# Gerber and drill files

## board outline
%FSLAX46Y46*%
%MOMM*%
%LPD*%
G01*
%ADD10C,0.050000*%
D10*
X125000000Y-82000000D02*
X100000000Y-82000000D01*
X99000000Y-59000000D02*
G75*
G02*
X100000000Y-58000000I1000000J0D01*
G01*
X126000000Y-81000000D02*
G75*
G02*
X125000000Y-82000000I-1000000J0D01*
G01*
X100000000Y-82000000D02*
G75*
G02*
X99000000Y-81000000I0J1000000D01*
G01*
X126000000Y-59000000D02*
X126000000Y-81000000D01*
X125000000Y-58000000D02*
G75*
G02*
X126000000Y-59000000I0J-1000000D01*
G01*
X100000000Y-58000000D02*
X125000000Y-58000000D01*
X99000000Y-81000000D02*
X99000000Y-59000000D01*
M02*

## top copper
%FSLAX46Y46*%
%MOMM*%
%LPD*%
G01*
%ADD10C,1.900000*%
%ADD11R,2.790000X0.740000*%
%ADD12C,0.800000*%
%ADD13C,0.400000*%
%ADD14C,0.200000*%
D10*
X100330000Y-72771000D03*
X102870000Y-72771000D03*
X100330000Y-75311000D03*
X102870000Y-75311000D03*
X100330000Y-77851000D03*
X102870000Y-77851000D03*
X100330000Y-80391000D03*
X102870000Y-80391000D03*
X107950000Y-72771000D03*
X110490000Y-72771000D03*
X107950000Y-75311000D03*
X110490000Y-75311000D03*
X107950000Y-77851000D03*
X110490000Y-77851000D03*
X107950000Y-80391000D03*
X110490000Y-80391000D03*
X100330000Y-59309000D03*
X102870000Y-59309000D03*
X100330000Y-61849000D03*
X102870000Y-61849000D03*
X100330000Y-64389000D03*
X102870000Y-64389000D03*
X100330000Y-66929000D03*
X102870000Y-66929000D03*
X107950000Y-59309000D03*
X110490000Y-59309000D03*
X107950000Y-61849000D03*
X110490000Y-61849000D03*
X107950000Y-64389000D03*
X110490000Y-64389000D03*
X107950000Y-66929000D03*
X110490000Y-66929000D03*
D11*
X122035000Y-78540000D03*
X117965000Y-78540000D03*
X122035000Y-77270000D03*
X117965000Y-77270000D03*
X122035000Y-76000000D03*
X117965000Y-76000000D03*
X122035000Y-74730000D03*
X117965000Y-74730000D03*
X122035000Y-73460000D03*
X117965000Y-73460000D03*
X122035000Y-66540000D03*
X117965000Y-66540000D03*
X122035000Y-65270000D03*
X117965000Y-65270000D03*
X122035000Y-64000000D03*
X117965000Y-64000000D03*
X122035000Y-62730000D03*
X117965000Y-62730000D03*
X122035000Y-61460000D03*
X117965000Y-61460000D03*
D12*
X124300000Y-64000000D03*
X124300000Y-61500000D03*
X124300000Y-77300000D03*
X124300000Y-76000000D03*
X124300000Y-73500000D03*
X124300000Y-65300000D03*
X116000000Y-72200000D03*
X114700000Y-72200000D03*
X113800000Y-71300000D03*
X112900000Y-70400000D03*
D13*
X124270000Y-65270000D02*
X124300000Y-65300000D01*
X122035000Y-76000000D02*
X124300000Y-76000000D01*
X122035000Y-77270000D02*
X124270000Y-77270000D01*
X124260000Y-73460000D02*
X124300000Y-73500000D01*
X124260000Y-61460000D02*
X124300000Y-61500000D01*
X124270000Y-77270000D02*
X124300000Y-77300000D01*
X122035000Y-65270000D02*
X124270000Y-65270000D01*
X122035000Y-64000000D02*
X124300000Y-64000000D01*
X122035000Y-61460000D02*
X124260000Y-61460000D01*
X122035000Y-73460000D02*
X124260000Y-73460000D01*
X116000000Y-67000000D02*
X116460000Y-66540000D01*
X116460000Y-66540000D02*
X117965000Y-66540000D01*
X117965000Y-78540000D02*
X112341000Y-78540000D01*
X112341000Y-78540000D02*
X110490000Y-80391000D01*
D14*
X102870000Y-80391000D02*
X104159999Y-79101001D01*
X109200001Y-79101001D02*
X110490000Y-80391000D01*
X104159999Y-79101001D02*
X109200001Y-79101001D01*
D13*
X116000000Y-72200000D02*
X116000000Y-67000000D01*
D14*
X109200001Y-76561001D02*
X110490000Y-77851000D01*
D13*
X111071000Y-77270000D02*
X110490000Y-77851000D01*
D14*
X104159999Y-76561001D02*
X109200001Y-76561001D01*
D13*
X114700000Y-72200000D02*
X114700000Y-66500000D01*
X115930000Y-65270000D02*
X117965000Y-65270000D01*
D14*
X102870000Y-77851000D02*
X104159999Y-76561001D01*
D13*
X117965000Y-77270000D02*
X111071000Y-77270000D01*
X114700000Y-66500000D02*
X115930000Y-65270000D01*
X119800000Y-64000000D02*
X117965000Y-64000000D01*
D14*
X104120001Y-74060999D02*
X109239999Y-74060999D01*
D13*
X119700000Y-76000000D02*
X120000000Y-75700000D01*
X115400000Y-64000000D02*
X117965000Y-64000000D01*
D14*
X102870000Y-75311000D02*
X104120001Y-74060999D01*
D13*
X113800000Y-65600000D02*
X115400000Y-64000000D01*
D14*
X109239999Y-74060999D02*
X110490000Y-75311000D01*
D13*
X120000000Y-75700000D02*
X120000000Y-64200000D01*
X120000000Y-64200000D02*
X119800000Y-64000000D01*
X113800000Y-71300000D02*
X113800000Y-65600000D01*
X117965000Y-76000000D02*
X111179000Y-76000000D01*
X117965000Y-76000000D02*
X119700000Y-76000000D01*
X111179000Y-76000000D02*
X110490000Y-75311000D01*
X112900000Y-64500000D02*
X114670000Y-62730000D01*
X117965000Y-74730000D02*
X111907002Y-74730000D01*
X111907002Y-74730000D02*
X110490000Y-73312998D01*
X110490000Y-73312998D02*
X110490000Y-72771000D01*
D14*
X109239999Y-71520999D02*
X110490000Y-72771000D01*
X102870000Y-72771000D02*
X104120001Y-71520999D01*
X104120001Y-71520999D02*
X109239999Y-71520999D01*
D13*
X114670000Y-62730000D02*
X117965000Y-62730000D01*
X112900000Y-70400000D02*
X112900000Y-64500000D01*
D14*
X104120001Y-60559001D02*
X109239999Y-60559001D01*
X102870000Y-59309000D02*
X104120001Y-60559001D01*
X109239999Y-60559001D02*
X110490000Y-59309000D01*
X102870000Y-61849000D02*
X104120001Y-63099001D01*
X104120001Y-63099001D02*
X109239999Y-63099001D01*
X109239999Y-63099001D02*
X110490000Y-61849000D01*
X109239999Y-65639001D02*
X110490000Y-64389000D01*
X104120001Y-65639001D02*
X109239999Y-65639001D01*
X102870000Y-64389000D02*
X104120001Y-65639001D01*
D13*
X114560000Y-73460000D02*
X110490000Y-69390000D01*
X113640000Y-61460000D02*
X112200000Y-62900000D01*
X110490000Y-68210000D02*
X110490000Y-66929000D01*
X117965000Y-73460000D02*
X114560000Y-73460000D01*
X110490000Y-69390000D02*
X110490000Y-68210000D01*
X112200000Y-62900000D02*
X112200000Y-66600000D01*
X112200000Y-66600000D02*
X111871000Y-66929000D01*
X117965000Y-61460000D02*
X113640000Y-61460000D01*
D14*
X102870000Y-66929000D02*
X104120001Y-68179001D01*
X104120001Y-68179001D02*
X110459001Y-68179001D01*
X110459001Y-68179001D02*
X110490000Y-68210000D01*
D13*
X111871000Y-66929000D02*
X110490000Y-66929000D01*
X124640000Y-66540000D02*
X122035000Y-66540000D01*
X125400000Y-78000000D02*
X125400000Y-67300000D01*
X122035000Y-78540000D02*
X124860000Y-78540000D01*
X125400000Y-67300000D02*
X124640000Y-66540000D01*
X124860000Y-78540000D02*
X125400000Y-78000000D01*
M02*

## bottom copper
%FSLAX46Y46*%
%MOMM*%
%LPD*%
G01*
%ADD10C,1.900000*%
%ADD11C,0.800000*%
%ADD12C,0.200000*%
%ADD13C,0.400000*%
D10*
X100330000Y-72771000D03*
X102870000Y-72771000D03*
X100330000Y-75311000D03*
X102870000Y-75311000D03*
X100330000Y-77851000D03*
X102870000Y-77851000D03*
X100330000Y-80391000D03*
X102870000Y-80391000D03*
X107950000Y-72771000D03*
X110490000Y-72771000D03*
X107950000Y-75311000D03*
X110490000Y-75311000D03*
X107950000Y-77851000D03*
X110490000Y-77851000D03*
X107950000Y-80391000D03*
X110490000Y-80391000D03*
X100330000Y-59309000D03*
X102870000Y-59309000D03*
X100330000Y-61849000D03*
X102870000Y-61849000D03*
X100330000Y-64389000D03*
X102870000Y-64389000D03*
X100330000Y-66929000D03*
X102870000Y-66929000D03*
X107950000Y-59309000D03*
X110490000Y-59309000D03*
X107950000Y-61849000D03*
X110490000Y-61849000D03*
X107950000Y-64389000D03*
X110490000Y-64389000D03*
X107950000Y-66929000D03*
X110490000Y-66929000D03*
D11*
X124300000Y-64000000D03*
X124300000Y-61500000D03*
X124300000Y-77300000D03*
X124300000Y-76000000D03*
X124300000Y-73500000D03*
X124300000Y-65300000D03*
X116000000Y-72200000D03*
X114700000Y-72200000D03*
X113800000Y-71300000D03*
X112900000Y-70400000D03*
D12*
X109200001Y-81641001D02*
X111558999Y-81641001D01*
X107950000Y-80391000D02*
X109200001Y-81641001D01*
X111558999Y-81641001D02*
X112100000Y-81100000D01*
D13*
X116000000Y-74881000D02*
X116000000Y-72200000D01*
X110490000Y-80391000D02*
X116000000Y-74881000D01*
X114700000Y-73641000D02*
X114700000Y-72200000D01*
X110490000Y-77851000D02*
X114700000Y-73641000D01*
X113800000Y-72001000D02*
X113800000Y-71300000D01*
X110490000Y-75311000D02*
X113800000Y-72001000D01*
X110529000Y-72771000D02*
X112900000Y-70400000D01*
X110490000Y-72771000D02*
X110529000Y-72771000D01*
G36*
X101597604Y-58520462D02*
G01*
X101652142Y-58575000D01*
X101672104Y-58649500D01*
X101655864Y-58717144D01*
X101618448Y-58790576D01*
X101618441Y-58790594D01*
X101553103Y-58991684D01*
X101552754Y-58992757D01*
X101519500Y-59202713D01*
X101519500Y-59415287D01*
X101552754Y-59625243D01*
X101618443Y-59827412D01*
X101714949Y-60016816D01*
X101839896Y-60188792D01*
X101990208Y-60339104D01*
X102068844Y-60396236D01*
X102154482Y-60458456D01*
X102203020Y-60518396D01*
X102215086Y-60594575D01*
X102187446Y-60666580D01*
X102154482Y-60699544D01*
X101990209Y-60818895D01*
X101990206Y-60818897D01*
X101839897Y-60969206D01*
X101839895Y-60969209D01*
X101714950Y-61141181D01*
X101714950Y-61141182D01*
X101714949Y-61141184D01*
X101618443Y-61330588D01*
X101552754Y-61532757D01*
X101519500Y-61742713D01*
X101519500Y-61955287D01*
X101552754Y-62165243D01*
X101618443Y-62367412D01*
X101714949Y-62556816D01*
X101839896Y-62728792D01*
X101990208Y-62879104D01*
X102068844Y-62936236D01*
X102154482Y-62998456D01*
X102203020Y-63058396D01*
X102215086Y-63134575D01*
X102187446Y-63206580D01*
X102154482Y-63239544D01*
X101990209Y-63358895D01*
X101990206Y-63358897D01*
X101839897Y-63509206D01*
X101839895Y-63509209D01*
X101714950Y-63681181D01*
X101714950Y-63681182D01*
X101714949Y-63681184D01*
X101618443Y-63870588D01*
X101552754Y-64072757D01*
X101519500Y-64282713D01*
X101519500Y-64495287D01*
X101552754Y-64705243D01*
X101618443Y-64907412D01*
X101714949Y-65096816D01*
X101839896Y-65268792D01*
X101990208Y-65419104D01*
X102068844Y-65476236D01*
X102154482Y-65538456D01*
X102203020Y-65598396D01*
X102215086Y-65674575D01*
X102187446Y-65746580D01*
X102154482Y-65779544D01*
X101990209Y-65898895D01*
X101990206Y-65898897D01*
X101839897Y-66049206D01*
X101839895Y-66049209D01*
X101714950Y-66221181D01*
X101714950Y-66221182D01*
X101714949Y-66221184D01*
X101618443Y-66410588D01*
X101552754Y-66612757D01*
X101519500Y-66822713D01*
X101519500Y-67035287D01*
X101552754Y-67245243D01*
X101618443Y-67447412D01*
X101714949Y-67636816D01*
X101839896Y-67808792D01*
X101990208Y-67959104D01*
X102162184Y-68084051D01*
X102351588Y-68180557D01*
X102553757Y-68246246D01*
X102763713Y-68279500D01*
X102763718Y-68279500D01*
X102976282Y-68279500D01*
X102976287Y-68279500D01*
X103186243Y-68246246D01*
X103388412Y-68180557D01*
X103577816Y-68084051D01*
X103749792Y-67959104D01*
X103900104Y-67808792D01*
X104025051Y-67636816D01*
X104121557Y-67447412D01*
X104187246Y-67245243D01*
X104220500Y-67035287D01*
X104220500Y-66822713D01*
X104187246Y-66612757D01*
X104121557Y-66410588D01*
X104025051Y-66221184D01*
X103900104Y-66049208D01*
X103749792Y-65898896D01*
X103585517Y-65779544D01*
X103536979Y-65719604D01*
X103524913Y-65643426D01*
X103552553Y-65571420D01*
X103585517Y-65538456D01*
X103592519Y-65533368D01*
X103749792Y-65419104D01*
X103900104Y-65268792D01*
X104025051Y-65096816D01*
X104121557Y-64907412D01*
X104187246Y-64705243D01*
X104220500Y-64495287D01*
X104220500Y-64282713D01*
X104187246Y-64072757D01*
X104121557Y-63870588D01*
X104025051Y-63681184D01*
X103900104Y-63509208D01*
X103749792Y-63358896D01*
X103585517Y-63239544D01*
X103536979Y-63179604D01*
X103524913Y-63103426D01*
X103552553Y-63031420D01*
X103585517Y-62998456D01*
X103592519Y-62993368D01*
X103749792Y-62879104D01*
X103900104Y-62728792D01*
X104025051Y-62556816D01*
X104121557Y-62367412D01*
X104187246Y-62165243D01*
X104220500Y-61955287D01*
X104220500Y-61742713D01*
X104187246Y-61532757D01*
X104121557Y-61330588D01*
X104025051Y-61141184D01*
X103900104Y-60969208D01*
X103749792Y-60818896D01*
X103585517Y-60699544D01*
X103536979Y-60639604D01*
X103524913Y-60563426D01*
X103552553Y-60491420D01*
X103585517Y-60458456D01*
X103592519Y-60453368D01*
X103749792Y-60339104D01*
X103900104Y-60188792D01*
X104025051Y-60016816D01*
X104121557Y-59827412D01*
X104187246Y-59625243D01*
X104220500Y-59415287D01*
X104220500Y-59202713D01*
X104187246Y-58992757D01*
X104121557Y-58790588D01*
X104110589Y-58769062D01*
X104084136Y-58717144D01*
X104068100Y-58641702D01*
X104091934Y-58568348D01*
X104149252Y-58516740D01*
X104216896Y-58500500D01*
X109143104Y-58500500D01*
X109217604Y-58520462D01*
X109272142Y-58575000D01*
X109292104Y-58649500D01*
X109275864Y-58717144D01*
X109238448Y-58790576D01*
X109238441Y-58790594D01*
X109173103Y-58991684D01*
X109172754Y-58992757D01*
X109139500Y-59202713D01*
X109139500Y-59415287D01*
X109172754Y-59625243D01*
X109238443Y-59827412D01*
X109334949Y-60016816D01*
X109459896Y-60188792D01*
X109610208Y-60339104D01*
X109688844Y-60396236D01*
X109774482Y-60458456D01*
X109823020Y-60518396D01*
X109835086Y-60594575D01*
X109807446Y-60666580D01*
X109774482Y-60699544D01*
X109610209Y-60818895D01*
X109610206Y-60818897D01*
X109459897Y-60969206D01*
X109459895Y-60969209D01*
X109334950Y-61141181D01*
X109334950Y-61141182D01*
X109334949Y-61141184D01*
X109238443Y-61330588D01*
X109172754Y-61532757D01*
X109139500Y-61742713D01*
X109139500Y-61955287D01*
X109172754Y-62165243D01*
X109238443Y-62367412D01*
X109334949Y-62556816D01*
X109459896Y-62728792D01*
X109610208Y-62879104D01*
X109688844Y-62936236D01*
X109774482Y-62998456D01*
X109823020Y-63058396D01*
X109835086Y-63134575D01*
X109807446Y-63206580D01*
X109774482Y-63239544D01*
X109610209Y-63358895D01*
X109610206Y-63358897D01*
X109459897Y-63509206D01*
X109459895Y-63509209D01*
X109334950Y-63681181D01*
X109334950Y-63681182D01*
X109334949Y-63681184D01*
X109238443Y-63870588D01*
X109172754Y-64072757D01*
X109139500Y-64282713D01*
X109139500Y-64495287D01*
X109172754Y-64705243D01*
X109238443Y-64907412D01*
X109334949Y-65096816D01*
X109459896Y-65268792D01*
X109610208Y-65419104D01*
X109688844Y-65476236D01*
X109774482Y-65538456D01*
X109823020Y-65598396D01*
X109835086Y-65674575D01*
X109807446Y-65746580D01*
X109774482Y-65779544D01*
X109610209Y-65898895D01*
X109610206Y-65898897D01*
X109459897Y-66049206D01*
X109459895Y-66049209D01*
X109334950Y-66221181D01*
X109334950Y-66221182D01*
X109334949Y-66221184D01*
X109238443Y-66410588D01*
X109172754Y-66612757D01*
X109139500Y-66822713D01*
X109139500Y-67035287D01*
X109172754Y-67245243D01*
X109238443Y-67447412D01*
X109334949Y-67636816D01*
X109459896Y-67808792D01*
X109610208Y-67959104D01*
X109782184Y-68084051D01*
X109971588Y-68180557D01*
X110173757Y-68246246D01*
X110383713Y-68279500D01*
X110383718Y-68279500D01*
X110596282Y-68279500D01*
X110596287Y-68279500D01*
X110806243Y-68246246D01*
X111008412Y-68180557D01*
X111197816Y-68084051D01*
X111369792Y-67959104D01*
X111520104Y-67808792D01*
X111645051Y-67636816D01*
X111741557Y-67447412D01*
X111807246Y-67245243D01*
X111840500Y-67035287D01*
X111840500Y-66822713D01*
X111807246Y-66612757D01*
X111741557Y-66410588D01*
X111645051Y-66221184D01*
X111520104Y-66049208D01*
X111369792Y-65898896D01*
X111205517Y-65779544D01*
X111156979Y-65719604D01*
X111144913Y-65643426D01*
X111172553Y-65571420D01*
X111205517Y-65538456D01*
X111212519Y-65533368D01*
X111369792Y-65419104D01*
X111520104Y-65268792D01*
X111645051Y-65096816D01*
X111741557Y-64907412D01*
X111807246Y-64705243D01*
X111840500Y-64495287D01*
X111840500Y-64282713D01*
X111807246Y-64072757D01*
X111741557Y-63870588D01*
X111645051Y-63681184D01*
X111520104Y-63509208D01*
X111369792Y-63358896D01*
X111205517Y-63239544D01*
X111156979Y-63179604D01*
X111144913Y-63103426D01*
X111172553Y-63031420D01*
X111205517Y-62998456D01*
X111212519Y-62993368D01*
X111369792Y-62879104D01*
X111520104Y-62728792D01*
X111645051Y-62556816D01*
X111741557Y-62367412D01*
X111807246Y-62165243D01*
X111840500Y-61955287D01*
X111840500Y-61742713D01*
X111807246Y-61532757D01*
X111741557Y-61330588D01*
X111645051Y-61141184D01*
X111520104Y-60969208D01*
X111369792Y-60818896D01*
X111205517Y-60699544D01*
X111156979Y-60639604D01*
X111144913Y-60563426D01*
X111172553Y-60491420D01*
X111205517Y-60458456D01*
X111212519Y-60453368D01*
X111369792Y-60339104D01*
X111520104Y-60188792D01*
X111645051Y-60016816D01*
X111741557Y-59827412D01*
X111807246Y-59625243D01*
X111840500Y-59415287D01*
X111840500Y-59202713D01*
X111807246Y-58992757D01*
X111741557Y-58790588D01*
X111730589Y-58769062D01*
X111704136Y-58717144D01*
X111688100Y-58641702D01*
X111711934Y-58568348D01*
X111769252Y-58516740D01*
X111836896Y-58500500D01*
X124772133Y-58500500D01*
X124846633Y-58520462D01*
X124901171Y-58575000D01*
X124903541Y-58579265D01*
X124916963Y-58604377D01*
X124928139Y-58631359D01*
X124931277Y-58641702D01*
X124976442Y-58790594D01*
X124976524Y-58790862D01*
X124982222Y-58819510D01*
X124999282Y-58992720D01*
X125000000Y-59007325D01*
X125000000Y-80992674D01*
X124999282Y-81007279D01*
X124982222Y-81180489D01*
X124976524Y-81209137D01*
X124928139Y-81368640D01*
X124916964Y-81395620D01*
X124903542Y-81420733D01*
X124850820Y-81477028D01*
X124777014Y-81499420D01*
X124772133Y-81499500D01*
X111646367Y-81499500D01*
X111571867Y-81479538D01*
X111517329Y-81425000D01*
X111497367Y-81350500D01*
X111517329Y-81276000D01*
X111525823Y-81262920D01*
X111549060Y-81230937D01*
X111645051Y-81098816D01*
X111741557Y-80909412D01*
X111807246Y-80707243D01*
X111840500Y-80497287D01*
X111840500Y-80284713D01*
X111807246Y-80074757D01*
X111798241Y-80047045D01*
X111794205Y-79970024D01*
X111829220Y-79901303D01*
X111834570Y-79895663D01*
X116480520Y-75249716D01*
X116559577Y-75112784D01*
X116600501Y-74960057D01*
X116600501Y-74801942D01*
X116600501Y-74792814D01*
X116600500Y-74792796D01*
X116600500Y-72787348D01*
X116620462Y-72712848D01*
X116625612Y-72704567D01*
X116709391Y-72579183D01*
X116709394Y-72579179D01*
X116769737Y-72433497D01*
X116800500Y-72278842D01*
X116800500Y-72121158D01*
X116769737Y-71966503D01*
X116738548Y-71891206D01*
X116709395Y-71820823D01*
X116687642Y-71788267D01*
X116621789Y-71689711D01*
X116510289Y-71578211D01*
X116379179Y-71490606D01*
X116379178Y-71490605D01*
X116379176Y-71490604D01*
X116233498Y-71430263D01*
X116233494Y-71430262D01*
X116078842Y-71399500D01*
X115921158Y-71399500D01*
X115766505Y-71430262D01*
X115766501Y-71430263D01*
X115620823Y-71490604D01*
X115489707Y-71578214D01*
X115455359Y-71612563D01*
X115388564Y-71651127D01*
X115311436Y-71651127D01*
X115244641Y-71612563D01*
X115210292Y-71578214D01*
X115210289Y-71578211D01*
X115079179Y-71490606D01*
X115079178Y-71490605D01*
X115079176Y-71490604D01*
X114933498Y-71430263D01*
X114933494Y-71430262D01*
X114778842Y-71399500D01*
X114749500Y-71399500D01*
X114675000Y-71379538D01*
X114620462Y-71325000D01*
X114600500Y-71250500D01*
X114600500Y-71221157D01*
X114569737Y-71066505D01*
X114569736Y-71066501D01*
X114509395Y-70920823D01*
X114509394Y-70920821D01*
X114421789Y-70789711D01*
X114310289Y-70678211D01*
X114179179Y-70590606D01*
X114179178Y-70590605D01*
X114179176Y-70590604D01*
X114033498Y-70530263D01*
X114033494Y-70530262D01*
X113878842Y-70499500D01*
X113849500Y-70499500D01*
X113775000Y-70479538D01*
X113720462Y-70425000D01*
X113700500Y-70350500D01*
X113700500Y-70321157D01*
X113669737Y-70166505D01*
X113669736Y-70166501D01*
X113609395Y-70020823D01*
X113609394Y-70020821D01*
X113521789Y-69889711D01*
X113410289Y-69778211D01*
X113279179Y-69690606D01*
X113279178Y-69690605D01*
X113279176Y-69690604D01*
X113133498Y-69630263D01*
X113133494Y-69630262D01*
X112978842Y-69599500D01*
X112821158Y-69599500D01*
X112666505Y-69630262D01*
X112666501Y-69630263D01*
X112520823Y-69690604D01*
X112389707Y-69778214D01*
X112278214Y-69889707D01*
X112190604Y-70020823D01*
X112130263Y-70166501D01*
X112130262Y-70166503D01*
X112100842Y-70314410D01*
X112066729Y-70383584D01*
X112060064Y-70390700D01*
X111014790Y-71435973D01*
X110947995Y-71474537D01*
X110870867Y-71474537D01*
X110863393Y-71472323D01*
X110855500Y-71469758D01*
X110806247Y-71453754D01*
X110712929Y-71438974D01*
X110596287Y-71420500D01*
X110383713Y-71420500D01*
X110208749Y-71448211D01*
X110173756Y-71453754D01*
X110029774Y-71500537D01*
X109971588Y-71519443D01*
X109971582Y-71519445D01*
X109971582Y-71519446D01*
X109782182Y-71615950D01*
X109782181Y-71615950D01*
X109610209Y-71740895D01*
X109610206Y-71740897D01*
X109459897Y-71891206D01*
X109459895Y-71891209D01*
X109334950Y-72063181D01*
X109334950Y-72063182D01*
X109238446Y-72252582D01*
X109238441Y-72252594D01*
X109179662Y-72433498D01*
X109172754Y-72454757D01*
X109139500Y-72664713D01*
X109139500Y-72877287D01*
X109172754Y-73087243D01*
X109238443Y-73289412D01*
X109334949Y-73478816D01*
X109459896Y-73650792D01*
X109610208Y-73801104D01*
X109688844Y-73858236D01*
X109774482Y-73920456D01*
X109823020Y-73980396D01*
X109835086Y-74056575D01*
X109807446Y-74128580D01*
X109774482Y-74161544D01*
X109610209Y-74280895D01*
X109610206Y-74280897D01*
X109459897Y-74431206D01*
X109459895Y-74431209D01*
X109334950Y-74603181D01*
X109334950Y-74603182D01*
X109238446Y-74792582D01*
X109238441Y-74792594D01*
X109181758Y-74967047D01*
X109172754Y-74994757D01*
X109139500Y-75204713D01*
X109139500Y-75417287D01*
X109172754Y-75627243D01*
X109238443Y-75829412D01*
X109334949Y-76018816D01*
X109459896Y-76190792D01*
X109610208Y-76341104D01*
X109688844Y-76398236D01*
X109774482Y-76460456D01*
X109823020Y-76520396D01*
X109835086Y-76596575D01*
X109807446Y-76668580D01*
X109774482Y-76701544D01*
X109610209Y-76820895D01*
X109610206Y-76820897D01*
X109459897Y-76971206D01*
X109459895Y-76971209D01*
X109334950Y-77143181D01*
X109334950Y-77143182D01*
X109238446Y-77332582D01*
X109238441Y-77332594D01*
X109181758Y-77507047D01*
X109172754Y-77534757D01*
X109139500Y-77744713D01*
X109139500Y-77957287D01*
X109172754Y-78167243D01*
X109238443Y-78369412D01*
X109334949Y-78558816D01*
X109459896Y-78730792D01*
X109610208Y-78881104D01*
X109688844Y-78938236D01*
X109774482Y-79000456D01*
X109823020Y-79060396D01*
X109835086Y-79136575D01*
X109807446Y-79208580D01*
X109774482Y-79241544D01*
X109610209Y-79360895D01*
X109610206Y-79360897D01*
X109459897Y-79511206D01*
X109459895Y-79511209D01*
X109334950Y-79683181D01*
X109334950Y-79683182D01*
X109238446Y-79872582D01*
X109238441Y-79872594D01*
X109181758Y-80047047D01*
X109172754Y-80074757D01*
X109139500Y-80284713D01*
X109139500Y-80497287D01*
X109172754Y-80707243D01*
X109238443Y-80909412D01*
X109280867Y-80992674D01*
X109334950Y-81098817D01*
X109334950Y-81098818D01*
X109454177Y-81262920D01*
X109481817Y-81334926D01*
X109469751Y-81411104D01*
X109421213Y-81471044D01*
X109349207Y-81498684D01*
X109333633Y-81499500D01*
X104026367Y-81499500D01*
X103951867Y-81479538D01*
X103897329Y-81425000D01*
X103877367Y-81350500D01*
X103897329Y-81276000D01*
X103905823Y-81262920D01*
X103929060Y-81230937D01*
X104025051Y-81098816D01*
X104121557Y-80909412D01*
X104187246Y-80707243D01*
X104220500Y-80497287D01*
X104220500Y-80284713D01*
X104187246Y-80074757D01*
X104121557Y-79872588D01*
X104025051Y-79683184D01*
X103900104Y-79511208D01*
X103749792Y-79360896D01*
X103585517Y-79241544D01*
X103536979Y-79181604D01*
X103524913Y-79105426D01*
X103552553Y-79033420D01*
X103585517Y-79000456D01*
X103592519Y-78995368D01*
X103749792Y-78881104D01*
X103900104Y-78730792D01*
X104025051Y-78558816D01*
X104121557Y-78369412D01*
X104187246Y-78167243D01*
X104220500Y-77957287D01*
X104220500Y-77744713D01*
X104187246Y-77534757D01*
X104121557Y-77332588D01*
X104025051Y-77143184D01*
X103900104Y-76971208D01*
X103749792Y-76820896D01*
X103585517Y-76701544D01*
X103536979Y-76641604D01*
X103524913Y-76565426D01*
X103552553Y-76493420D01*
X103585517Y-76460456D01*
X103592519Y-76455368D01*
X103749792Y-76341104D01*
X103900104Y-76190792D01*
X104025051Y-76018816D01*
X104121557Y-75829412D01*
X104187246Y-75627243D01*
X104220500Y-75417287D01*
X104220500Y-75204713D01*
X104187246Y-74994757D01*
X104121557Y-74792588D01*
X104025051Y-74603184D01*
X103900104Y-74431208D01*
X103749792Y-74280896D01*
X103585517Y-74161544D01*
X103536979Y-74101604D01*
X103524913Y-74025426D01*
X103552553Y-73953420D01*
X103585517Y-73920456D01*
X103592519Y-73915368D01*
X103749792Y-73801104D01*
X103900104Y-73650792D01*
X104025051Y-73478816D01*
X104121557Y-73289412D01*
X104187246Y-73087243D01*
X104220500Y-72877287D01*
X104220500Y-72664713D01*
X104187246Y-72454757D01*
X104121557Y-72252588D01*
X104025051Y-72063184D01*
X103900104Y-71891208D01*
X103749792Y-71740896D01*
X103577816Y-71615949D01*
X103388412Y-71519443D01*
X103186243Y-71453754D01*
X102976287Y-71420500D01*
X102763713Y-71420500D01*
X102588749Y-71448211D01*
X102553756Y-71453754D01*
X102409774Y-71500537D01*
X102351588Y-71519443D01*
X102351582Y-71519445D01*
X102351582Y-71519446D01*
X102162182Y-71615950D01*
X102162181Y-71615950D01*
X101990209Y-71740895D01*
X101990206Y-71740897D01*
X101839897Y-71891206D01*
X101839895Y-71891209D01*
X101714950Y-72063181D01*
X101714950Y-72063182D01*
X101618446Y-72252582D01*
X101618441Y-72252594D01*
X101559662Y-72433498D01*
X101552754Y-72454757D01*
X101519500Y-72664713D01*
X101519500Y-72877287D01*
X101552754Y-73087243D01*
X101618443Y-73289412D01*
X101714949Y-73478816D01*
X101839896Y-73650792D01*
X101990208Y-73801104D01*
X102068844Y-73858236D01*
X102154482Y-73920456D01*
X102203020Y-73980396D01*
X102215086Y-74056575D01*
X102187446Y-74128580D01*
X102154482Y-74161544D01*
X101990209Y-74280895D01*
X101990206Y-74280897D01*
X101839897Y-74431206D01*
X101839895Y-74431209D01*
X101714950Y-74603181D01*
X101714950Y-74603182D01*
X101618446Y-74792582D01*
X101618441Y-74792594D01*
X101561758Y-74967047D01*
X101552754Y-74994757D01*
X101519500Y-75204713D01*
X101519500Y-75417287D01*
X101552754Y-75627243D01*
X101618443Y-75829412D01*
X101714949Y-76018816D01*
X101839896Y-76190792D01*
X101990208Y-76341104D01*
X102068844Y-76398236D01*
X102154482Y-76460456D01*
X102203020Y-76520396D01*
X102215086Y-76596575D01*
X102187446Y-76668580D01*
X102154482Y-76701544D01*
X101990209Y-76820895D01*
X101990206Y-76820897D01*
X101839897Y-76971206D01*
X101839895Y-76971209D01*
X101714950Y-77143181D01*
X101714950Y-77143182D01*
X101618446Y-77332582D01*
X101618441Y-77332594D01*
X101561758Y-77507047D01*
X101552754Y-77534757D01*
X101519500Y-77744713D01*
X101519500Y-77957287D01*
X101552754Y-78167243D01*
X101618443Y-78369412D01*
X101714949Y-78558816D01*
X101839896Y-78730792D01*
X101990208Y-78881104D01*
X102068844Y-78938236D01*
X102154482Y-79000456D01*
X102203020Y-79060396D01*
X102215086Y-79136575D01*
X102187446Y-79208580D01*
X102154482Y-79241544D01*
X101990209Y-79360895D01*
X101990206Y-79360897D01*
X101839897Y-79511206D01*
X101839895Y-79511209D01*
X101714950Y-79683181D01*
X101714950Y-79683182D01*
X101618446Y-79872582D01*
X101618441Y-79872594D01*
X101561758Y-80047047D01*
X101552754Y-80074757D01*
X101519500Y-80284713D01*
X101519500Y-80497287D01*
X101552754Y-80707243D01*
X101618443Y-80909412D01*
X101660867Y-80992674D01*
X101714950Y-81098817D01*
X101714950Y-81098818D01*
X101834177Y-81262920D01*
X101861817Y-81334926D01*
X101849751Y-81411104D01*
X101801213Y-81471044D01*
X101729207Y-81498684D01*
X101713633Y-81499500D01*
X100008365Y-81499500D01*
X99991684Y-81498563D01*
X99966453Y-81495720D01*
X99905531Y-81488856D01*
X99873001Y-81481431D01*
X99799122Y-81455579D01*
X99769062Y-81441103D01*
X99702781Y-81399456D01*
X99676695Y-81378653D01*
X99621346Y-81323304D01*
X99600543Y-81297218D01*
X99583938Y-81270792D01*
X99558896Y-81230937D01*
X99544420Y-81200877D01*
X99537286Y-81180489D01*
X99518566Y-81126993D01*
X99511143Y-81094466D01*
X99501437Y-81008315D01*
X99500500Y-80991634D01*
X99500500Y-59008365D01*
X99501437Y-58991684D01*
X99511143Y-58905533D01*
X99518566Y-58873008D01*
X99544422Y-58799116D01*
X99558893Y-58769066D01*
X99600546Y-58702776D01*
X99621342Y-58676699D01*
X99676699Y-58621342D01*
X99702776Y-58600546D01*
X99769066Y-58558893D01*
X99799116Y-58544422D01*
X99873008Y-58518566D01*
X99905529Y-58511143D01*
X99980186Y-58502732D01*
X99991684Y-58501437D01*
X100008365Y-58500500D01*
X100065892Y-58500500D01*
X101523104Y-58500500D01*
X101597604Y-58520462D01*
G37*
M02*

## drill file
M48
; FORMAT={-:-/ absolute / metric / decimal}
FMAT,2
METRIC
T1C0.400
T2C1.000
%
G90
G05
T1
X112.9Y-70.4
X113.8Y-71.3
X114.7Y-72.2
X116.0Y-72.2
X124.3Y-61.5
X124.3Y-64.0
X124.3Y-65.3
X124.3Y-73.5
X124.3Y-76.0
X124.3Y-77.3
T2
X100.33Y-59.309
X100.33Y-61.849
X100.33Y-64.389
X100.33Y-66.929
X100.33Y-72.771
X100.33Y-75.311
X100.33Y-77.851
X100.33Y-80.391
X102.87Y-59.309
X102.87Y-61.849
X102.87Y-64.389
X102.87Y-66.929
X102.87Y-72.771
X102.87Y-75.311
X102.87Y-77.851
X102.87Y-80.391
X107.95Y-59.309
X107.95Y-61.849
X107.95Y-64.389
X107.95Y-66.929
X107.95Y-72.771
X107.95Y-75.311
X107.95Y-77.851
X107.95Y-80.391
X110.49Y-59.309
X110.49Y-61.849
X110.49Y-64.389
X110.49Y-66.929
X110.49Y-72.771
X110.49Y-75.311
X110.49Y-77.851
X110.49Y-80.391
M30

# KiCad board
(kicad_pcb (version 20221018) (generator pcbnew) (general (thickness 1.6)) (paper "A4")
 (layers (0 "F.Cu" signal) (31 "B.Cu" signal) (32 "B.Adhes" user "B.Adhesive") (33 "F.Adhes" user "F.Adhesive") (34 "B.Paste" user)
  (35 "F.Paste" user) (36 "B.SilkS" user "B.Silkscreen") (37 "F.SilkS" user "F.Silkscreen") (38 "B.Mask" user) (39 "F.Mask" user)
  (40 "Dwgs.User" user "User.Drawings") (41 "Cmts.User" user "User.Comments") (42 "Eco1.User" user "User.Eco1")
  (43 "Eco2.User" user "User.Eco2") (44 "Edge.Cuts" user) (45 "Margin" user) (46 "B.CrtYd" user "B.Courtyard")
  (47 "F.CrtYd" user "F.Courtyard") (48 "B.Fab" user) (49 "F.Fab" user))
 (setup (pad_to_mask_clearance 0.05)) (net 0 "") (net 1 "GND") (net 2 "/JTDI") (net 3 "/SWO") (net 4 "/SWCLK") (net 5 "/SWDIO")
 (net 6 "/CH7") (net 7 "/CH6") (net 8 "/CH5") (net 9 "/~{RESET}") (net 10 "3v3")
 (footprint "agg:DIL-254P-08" (layer "F.Cu") (at 101.6 76.581 -90)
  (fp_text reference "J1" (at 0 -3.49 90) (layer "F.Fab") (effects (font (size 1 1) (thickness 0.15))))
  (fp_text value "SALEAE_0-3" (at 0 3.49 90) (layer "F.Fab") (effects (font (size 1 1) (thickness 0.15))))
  (pad "1" thru_hole circle (at -3.81 1.27 270) (size 1.9 1.9) (drill 1) (layers "*.Cu" "*.Mask" "F.SilkS") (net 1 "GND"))
  (pad "2" thru_hole circle (at -3.81 -1.27 270) (size 1.9 1.9) (drill 1) (layers "*.Cu" "*.Mask" "F.SilkS") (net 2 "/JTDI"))
  (pad "3" thru_hole circle (at -1.27 1.27 270) (size 1.9 1.9) (drill 1) (layers "*.Cu" "*.Mask" "F.SilkS") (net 1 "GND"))
  (pad "4" thru_hole circle (at -1.27 -1.27 270) (size 1.9 1.9) (drill 1) (layers "*.Cu" "*.Mask" "F.SilkS") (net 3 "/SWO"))
  (pad "5" thru_hole circle (at 1.27 1.27 270) (size 1.9 1.9) (drill 1) (layers "*.Cu" "*.Mask" "F.SilkS") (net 1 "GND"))
  (pad "6" thru_hole circle (at 1.27 -1.27 270) (size 1.9 1.9) (drill 1) (layers "*.Cu" "*.Mask" "F.SilkS") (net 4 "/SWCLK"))
  (pad "7" thru_hole circle (at 3.81 1.27 270) (size 1.9 1.9) (drill 1) (layers "*.Cu" "*.Mask" "F.SilkS") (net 1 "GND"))
  (pad "8" thru_hole circle (at 3.81 -1.27 270) (size 1.9 1.9) (drill 1) (layers "*.Cu" "*.Mask" "F.SilkS") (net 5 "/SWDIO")))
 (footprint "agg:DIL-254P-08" (layer "F.Cu") (at 109.22 76.581 -90)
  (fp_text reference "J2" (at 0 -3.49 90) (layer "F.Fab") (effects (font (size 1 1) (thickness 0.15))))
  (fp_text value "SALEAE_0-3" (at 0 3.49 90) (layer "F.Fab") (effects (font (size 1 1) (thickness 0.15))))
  (pad "1" thru_hole circle (at -3.81 1.27 270) (size 1.9 1.9) (drill 1) (layers "*.Cu" "*.Mask" "F.SilkS") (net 1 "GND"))
  (pad "2" thru_hole circle (at -3.81 -1.27 270) (size 1.9 1.9) (drill 1) (layers "*.Cu" "*.Mask" "F.SilkS") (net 2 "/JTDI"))
  (pad "3" thru_hole circle (at -1.27 1.27 270) (size 1.9 1.9) (drill 1) (layers "*.Cu" "*.Mask" "F.SilkS") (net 1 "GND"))
  (pad "4" thru_hole circle (at -1.27 -1.27 270) (size 1.9 1.9) (drill 1) (layers "*.Cu" "*.Mask" "F.SilkS") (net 3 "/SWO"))
  (pad "5" thru_hole circle (at 1.27 1.27 270) (size 1.9 1.9) (drill 1) (layers "*.Cu" "*.Mask" "F.SilkS") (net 1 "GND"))
  (pad "6" thru_hole circle (at 1.27 -1.27 270) (size 1.9 1.9) (drill 1) (layers "*.Cu" "*.Mask" "F.SilkS") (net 4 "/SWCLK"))
  (pad "7" thru_hole circle (at 3.81 1.27 270) (size 1.9 1.9) (drill 1) (layers "*.Cu" "*.Mask" "F.SilkS") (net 1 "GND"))
  (pad "8" thru_hole circle (at 3.81 -1.27 270) (size 1.9 1.9) (drill 1) (layers "*.Cu" "*.Mask" "F.SilkS") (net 5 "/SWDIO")))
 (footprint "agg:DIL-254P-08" (layer "F.Cu") (at 101.6 63.119 -90)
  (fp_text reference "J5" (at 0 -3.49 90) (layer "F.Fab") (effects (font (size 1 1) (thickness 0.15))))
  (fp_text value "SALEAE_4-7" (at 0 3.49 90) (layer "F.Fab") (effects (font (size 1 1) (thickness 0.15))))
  (pad "1" thru_hole circle (at -3.81 1.27 270) (size 1.9 1.9) (drill 1) (layers "*.Cu" "*.Mask" "F.SilkS") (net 1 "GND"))
  (pad "2" thru_hole circle (at -3.81 -1.27 270) (size 1.9 1.9) (drill 1) (layers "*.Cu" "*.Mask" "F.SilkS") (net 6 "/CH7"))
  (pad "3" thru_hole circle (at -1.27 1.27 270) (size 1.9 1.9) (drill 1) (layers "*.Cu" "*.Mask" "F.SilkS") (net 1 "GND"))
  (pad "4" thru_hole circle (at -1.27 -1.27 270) (size 1.9 1.9) (drill 1) (layers "*.Cu" "*.Mask" "F.SilkS") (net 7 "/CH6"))
  (pad "5" thru_hole circle (at 1.27 1.27 270) (size 1.9 1.9) (drill 1) (layers "*.Cu" "*.Mask" "F.SilkS") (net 1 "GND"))
  (pad "6" thru_hole circle (at 1.27 -1.27 270) (size 1.9 1.9) (drill 1) (layers "*.Cu" "*.Mask" "F.SilkS") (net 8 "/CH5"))
  (pad "7" thru_hole circle (at 3.81 1.27 270) (size 1.9 1.9) (drill 1) (layers "*.Cu" "*.Mask" "F.SilkS") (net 1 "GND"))
  (pad "8" thru_hole circle (at 3.81 -1.27 270) (size 1.9 1.9) (drill 1) (layers "*.Cu" "*.Mask" "F.SilkS") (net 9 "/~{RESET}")))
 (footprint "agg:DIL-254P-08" (layer "F.Cu") (at 109.22 63.119 -90)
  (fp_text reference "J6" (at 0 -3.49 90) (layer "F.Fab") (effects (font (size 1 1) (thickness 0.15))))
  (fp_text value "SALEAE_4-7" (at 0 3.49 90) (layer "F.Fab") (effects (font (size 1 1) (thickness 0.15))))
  (pad "1" thru_hole circle (at -3.81 1.27 270) (size 1.9 1.9) (drill 1) (layers "*.Cu" "*.Mask" "F.SilkS") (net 1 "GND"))
  (pad "2" thru_hole circle (at -3.81 -1.27 270) (size 1.9 1.9) (drill 1) (layers "*.Cu" "*.Mask" "F.SilkS") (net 6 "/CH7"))
  (pad "3" thru_hole circle (at -1.27 1.27 270) (size 1.9 1.9) (drill 1) (layers "*.Cu" "*.Mask" "F.SilkS") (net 1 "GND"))
  (pad "4" thru_hole circle (at -1.27 -1.27 270) (size 1.9 1.9) (drill 1) (layers "*.Cu" "*.Mask" "F.SilkS") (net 7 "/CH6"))
  (pad "5" thru_hole circle (at 1.27 1.27 270) (size 1.9 1.9) (drill 1) (layers "*.Cu" "*.Mask" "F.SilkS") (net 1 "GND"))
  (pad "6" thru_hole circle (at 1.27 -1.27 270) (size 1.9 1.9) (drill 1) (layers "*.Cu" "*.Mask" "F.SilkS") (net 8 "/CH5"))
  (pad "7" thru_hole circle (at 3.81 1.27 270) (size 1.9 1.9) (drill 1) (layers "*.Cu" "*.Mask" "F.SilkS") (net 1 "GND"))
  (pad "8" thru_hole circle (at 3.81 -1.27 270) (size 1.9 1.9) (drill 1) (layers "*.Cu" "*.Mask" "F.SilkS") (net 9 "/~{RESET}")))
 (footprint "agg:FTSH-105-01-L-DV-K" (layer "F.Cu") (at 120 76 90)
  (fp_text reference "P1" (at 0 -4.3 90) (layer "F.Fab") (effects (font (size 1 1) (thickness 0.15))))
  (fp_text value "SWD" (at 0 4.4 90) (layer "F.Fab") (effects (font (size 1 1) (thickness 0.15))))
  (pad "1" smd rect (at -2.54 2.035 90) (size 0.74 2.79) (layers "F.Cu" "F.Paste" "F.Mask") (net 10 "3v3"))
  (pad "2" smd rect (at -2.54 -2.035 90) (size 0.74 2.79) (layers "F.Cu" "F.Paste" "F.Mask") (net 5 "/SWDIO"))
  (pad "3" smd rect (at -1.27 2.035 90) (size 0.74 2.79) (layers "F.Cu" "F.Paste" "F.Mask") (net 1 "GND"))
  (pad "4" smd rect (at -1.27 -2.035 90) (size 0.74 2.79) (layers "F.Cu" "F.Paste" "F.Mask") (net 4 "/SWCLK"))
  (pad "5" smd rect (at 0 2.035 90) (size 0.74 2.79) (layers "F.Cu" "F.Paste" "F.Mask") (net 1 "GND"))
  (pad "6" smd rect (at 0 -2.035 90) (size 0.74 2.79) (layers "F.Cu" "F.Paste" "F.Mask") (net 3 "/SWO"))
  (pad "7" smd rect (at 1.27 2.035 90) (size 0.74 2.79) (layers "F.Cu" "F.Paste" "F.Mask"))
  (pad "8" smd rect (at 1.27 -2.035 90) (size 0.74 2.79) (layers "F.Cu" "F.Paste" "F.Mask") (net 2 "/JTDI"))
  (pad "9" smd rect (at 2.54 2.035 90) (size 0.74 2.79) (layers "F.Cu" "F.Paste" "F.Mask") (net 1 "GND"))
  (pad "10" smd rect (at 2.54 -2.035 90) (size 0.74 2.79) (layers "F.Cu" "F.Paste" "F.Mask") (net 9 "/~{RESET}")))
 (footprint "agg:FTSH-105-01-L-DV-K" (layer "F.Cu") (at 120 64 90)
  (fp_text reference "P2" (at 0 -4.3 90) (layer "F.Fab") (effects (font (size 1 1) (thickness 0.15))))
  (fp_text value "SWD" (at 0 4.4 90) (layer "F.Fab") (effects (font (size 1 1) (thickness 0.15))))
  (pad "1" smd rect (at -2.54 2.035 90) (size 0.74 2.79) (layers "F.Cu" "F.Paste" "F.Mask") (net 10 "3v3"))
  (pad "2" smd rect (at -2.54 -2.035 90) (size 0.74 2.79) (layers "F.Cu" "F.Paste" "F.Mask") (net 5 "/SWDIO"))
  (pad "3" smd rect (at -1.27 2.035 90) (size 0.74 2.79) (layers "F.Cu" "F.Paste" "F.Mask") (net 1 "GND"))
  (pad "4" smd rect (at -1.27 -2.035 90) (size 0.74 2.79) (layers "F.Cu" "F.Paste" "F.Mask") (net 4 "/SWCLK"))
  (pad "5" smd rect (at 0 2.035 90) (size 0.74 2.79) (layers "F.Cu" "F.Paste" "F.Mask") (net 1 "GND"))
  (pad "6" smd rect (at 0 -2.035 90) (size 0.74 2.79) (layers "F.Cu" "F.Paste" "F.Mask") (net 3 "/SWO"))
  (pad "7" smd rect (at 1.27 2.035 90) (size 0.74 2.79) (layers "F.Cu" "F.Paste" "F.Mask"))
  (pad "8" smd rect (at 1.27 -2.035 90) (size 0.74 2.79) (layers "F.Cu" "F.Paste" "F.Mask") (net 2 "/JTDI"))
  (pad "9" smd rect (at 2.54 2.035 90) (size 0.74 2.79) (layers "F.Cu" "F.Paste" "F.Mask") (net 1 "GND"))
  (pad "10" smd rect (at 2.54 -2.035 90) (size 0.74 2.79) (layers "F.Cu" "F.Paste" "F.Mask") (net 9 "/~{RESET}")))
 (gr_line (start 125 82) (end 100 82) (stroke (width 0.05) (type solid)) (layer "Edge.Cuts"))
 (gr_arc (start 99 59) (mid 99.292893 58.292893) (end 100 58) (stroke (width 0.05) (type solid)) (layer "Edge.Cuts"))
 (gr_arc (start 126 81) (mid 125.707107 81.707107) (end 125 82) (stroke (width 0.05) (type solid)) (layer "Edge.Cuts"))
 (gr_arc (start 100 82) (mid 99.292893 81.707107) (end 99 81) (stroke (width 0.05) (type solid)) (layer "Edge.Cuts"))
 (gr_line (start 126 59) (end 126 81) (stroke (width 0.05) (type solid)) (layer "Edge.Cuts"))
 (gr_arc (start 125 58) (mid 125.707107 58.292893) (end 126 59) (stroke (width 0.05) (type solid)) (layer "Edge.Cuts"))
 (gr_line (start 100 58) (end 125 58) (stroke (width 0.05) (type solid)) (layer "Edge.Cuts"))
 (gr_line (start 99 81) (end 99 59) (stroke (width 0.05) (type solid)) (layer "Edge.Cuts"))
 (segment (start 124.27 65.27) (end 124.3 65.3) (width 0.4) (layer "F.Cu") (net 1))
 (segment (start 122.035 76) (end 124.3 76) (width 0.4) (layer "F.Cu") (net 1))
 (segment (start 122.035 77.27) (end 124.27 77.27) (width 0.4) (layer "F.Cu") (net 1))
 (segment (start 124.26 73.46) (end 124.3 73.5) (width 0.4) (layer "F.Cu") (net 1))
 (segment (start 124.26 61.46) (end 124.3 61.5) (width 0.4) (layer "F.Cu") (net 1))
 (segment (start 124.27 77.27) (end 124.3 77.3) (width 0.4) (layer "F.Cu") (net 1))
 (segment (start 122.035 65.27) (end 124.27 65.27) (width 0.4) (layer "F.Cu") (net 1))
 (segment (start 122.035 64) (end 124.3 64) (width 0.4) (layer "F.Cu") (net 1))
 (segment (start 122.035 61.46) (end 124.26 61.46) (width 0.4) (layer "F.Cu") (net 1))
 (segment (start 122.035 73.46) (end 124.26 73.46) (width 0.4) (layer "F.Cu") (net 1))
 (via (at 124.3 64) (size 0.8) (drill 0.4) (layers "F.Cu" "B.Cu") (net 1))
 (via (at 124.3 61.5) (size 0.8) (drill 0.4) (layers "F.Cu" "B.Cu") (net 1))
 (via (at 124.3 77.3) (size 0.8) (drill 0.4) (layers "F.Cu" "B.Cu") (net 1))
 (via (at 124.3 76) (size 0.8) (drill 0.4) (layers "F.Cu" "B.Cu") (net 1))
 (via (at 124.3 73.5) (size 0.8) (drill 0.4) (layers "F.Cu" "B.Cu") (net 1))
 (via (at 124.3 65.3) (size 0.8) (drill 0.4) (layers "F.Cu" "B.Cu") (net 1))
 (segment (start 109.200001 81.641001) (end 111.558999 81.641001) (width 0.2) (layer "B.Cu") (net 1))
 (segment (start 107.95 80.391) (end 109.200001 81.641001) (width 0.2) (layer "B.Cu") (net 1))
 (segment (start 111.558999 81.641001) (end 112.1 81.1) (width 0.2) (layer "B.Cu") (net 1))
 (segment (start 116 67) (end 116.46 66.54) (width 0.4) (layer "F.Cu") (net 5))
 (segment (start 116.46 66.54) (end 117.965 66.54) (width 0.4) (layer "F.Cu") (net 5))
 (segment (start 117.965 78.54) (end 112.341 78.54) (width 0.4) (layer "F.Cu") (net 5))
 (segment (start 112.341 78.54) (end 110.49 80.391) (width 0.4) (layer "F.Cu") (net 5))
 (segment (start 102.87 80.391) (end 104.159999 79.101001) (width 0.2) (layer "F.Cu") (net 5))
 (segment (start 109.200001 79.101001) (end 110.49 80.391) (width 0.2) (layer "F.Cu") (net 5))
 (segment (start 104.159999 79.101001) (end 109.200001 79.101001) (width 0.2) (layer "F.Cu") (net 5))
 (segment (start 116 72.2) (end 116 67) (width 0.4) (layer "F.Cu") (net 5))
 (via (at 116 72.2) (size 0.8) (drill 0.4) (layers "F.Cu" "B.Cu") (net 5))
 (segment (start 116 74.881) (end 116 72.2) (width 0.4) (layer "B.Cu") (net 5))
 (segment (start 110.49 80.391) (end 116 74.881) (width 0.4) (layer "B.Cu") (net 5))
 (segment (start 109.200001 76.561001) (end 110.49 77.851) (width 0.2) (layer "F.Cu") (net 4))
 (segment (start 111.071 77.27) (end 110.49 77.851) (width 0.4) (layer "F.Cu") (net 4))
 (segment (start 104.159999 76.561001) (end 109.200001 76.561001) (width 0.2) (layer "F.Cu") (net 4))
 (segment (start 114.7 72.2) (end 114.7 66.5) (width 0.4) (layer "F.Cu") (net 4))
 (segment (start 115.93 65.27) (end 117.965 65.27) (width 0.4) (layer "F.Cu") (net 4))
 (segment (start 102.87 77.851) (end 104.159999 76.561001) (width 0.2) (layer "F.Cu") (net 4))
 (segment (start 117.965 77.27) (end 111.071 77.27) (width 0.4) (layer "F.Cu") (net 4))
 (segment (start 114.7 66.5) (end 115.93 65.27) (width 0.4) (layer "F.Cu") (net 4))
 (via (at 114.7 72.2) (size 0.8) (drill 0.4) (layers "F.Cu" "B.Cu") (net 4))
 (segment (start 114.7 73.641) (end 114.7 72.2) (width 0.4) (layer "B.Cu") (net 4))
 (segment (start 110.49 77.851) (end 114.7 73.641) (width 0.4) (layer "B.Cu") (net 4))
 (segment (start 119.8 64) (end 117.965 64) (width 0.4) (layer "F.Cu") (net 3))
 (segment (start 104.120001 74.060999) (end 109.239999 74.060999) (width 0.2) (layer "F.Cu") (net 3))
 (segment (start 119.7 76) (end 120 75.7) (width 0.4) (layer "F.Cu") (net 3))
 (segment (start 115.4 64) (end 117.965 64) (width 0.4) (layer "F.Cu") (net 3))
 (segment (start 102.87 75.311) (end 104.120001 74.060999) (width 0.2) (layer "F.Cu") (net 3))
 (segment (start 113.8 65.6) (end 115.4 64) (width 0.4) (layer "F.Cu") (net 3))
 (segment (start 109.239999 74.060999) (end 110.49 75.311) (width 0.2) (layer "F.Cu") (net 3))
 (segment (start 120 75.7) (end 120 64.2) (width 0.4) (layer "F.Cu") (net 3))
 (segment (start 120 64.2) (end 119.8 64) (width 0.4) (layer "F.Cu") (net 3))
 (segment (start 113.8 71.3) (end 113.8 65.6) (width 0.4) (layer "F.Cu") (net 3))
 (segment (start 117.965 76) (end 111.179 76) (width 0.4) (layer "F.Cu") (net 3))
 (segment (start 117.965 76) (end 119.7 76) (width 0.4) (layer "F.Cu") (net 3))
 (segment (start 111.179 76) (end 110.49 75.311) (width 0.4) (layer "F.Cu") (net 3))
 (via (at 113.8 71.3) (size 0.8) (drill 0.4) (layers "F.Cu" "B.Cu") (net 3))
 (segment (start 113.8 72.001) (end 113.8 71.3) (width 0.4) (layer "B.Cu") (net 3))
 (segment (start 110.49 75.311) (end 113.8 72.001) (width 0.4) (layer "B.Cu") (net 3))
 (segment (start 112.9 64.5) (end 114.67 62.73) (width 0.4) (layer "F.Cu") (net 2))
 (segment (start 117.965 74.73) (end 111.907002 74.73) (width 0.4) (layer "F.Cu") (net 2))
 (segment (start 111.907002 74.73) (end 110.49 73.312998) (width 0.4) (layer "F.Cu") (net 2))
 (segment (start 110.49 73.312998) (end 110.49 72.771) (width 0.4) (layer "F.Cu") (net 2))
 (segment (start 109.239999 71.520999) (end 110.49 72.771) (width 0.2) (layer "F.Cu") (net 2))
 (segment (start 102.87 72.771) (end 104.120001 71.520999) (width 0.2) (layer "F.Cu") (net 2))
 (segment (start 104.120001 71.520999) (end 109.239999 71.520999) (width 0.2) (layer "F.Cu") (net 2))
 (segment (start 114.67 62.73) (end 117.965 62.73) (width 0.4) (layer "F.Cu") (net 2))
 (segment (start 112.9 70.4) (end 112.9 64.5) (width 0.4) (layer "F.Cu") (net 2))
 (via (at 112.9 70.4) (size 0.8) (drill 0.4) (layers "F.Cu" "B.Cu") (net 2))
 (segment (start 110.529 72.771) (end 112.9 70.4) (width 0.4) (layer "B.Cu") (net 2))
 (segment (start 110.49 72.771) (end 110.529 72.771) (width 0.4) (layer "B.Cu") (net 2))
 (segment (start 104.120001 60.559001) (end 109.239999 60.559001) (width 0.2) (layer "F.Cu") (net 6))
 (segment (start 102.87 59.309) (end 104.120001 60.559001) (width 0.2) (layer "F.Cu") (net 6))
 (segment (start 109.239999 60.559001) (end 110.49 59.309) (width 0.2) (layer "F.Cu") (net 6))
 (segment (start 102.87 61.849) (end 104.120001 63.099001) (width 0.2) (layer "F.Cu") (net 7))
 (segment (start 104.120001 63.099001) (end 109.239999 63.099001) (width 0.2) (layer "F.Cu") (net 7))
 (segment (start 109.239999 63.099001) (end 110.49 61.849) (width 0.2) (layer "F.Cu") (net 7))
 (segment (start 109.239999 65.639001) (end 110.49 64.389) (width 0.2) (layer "F.Cu") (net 8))
 (segment (start 104.120001 65.639001) (end 109.239999 65.639001) (width 0.2) (layer "F.Cu") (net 8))
 (segment (start 102.87 64.389) (end 104.120001 65.639001) (width 0.2) (layer "F.Cu") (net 8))
 (segment (start 114.56 73.46) (end 110.49 69.39) (width 0.4) (layer "F.Cu") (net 9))
 (segment (start 113.64 61.46) (end 112.2 62.9) (width 0.4) (layer "F.Cu") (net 9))
 (segment (start 110.49 68.21) (end 110.49 66.929) (width 0.4) (layer "F.Cu") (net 9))
 (segment (start 117.965 73.46) (end 114.56 73.46) (width 0.4) (layer "F.Cu") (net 9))
 (segment (start 110.49 69.39) (end 110.49 68.21) (width 0.4) (layer "F.Cu") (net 9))
 (segment (start 112.2 62.9) (end 112.2 66.6) (width 0.4) (layer "F.Cu") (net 9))
 (segment (start 112.2 66.6) (end 111.871 66.929) (width 0.4) (layer "F.Cu") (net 9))
 (segment (start 117.965 61.46) (end 113.64 61.46) (width 0.4) (layer "F.Cu") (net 9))
 (segment (start 102.87 66.929) (end 104.120001 68.179001) (width 0.2) (layer "F.Cu") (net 9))
 (segment (start 104.120001 68.179001) (end 110.459001 68.179001) (width 0.2) (layer "F.Cu") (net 9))
 (segment (start 110.459001 68.179001) (end 110.49 68.21) (width 0.2) (layer "F.Cu") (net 9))
 (segment (start 111.871 66.929) (end 110.49 66.929) (width 0.4) (layer "F.Cu") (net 9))
 (segment (start 124.64 66.54) (end 122.035 66.54) (width 0.4) (layer "F.Cu") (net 10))
 (segment (start 125.4 78) (end 125.4 67.3) (width 0.4) (layer "F.Cu") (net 10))
 (segment (start 122.035 78.54) (end 124.86 78.54) (width 0.4) (layer "F.Cu") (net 10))
 (segment (start 125.4 67.3) (end 124.64 66.54) (width 0.4) (layer "F.Cu") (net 10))
 (segment (start 124.86 78.54) (end 125.4 78) (width 0.4) (layer "F.Cu") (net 10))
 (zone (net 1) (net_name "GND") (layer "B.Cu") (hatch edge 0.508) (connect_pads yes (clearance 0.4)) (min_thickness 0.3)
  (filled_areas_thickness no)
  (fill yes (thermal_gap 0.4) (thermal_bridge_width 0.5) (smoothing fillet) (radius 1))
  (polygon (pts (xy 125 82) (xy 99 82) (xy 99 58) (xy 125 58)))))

